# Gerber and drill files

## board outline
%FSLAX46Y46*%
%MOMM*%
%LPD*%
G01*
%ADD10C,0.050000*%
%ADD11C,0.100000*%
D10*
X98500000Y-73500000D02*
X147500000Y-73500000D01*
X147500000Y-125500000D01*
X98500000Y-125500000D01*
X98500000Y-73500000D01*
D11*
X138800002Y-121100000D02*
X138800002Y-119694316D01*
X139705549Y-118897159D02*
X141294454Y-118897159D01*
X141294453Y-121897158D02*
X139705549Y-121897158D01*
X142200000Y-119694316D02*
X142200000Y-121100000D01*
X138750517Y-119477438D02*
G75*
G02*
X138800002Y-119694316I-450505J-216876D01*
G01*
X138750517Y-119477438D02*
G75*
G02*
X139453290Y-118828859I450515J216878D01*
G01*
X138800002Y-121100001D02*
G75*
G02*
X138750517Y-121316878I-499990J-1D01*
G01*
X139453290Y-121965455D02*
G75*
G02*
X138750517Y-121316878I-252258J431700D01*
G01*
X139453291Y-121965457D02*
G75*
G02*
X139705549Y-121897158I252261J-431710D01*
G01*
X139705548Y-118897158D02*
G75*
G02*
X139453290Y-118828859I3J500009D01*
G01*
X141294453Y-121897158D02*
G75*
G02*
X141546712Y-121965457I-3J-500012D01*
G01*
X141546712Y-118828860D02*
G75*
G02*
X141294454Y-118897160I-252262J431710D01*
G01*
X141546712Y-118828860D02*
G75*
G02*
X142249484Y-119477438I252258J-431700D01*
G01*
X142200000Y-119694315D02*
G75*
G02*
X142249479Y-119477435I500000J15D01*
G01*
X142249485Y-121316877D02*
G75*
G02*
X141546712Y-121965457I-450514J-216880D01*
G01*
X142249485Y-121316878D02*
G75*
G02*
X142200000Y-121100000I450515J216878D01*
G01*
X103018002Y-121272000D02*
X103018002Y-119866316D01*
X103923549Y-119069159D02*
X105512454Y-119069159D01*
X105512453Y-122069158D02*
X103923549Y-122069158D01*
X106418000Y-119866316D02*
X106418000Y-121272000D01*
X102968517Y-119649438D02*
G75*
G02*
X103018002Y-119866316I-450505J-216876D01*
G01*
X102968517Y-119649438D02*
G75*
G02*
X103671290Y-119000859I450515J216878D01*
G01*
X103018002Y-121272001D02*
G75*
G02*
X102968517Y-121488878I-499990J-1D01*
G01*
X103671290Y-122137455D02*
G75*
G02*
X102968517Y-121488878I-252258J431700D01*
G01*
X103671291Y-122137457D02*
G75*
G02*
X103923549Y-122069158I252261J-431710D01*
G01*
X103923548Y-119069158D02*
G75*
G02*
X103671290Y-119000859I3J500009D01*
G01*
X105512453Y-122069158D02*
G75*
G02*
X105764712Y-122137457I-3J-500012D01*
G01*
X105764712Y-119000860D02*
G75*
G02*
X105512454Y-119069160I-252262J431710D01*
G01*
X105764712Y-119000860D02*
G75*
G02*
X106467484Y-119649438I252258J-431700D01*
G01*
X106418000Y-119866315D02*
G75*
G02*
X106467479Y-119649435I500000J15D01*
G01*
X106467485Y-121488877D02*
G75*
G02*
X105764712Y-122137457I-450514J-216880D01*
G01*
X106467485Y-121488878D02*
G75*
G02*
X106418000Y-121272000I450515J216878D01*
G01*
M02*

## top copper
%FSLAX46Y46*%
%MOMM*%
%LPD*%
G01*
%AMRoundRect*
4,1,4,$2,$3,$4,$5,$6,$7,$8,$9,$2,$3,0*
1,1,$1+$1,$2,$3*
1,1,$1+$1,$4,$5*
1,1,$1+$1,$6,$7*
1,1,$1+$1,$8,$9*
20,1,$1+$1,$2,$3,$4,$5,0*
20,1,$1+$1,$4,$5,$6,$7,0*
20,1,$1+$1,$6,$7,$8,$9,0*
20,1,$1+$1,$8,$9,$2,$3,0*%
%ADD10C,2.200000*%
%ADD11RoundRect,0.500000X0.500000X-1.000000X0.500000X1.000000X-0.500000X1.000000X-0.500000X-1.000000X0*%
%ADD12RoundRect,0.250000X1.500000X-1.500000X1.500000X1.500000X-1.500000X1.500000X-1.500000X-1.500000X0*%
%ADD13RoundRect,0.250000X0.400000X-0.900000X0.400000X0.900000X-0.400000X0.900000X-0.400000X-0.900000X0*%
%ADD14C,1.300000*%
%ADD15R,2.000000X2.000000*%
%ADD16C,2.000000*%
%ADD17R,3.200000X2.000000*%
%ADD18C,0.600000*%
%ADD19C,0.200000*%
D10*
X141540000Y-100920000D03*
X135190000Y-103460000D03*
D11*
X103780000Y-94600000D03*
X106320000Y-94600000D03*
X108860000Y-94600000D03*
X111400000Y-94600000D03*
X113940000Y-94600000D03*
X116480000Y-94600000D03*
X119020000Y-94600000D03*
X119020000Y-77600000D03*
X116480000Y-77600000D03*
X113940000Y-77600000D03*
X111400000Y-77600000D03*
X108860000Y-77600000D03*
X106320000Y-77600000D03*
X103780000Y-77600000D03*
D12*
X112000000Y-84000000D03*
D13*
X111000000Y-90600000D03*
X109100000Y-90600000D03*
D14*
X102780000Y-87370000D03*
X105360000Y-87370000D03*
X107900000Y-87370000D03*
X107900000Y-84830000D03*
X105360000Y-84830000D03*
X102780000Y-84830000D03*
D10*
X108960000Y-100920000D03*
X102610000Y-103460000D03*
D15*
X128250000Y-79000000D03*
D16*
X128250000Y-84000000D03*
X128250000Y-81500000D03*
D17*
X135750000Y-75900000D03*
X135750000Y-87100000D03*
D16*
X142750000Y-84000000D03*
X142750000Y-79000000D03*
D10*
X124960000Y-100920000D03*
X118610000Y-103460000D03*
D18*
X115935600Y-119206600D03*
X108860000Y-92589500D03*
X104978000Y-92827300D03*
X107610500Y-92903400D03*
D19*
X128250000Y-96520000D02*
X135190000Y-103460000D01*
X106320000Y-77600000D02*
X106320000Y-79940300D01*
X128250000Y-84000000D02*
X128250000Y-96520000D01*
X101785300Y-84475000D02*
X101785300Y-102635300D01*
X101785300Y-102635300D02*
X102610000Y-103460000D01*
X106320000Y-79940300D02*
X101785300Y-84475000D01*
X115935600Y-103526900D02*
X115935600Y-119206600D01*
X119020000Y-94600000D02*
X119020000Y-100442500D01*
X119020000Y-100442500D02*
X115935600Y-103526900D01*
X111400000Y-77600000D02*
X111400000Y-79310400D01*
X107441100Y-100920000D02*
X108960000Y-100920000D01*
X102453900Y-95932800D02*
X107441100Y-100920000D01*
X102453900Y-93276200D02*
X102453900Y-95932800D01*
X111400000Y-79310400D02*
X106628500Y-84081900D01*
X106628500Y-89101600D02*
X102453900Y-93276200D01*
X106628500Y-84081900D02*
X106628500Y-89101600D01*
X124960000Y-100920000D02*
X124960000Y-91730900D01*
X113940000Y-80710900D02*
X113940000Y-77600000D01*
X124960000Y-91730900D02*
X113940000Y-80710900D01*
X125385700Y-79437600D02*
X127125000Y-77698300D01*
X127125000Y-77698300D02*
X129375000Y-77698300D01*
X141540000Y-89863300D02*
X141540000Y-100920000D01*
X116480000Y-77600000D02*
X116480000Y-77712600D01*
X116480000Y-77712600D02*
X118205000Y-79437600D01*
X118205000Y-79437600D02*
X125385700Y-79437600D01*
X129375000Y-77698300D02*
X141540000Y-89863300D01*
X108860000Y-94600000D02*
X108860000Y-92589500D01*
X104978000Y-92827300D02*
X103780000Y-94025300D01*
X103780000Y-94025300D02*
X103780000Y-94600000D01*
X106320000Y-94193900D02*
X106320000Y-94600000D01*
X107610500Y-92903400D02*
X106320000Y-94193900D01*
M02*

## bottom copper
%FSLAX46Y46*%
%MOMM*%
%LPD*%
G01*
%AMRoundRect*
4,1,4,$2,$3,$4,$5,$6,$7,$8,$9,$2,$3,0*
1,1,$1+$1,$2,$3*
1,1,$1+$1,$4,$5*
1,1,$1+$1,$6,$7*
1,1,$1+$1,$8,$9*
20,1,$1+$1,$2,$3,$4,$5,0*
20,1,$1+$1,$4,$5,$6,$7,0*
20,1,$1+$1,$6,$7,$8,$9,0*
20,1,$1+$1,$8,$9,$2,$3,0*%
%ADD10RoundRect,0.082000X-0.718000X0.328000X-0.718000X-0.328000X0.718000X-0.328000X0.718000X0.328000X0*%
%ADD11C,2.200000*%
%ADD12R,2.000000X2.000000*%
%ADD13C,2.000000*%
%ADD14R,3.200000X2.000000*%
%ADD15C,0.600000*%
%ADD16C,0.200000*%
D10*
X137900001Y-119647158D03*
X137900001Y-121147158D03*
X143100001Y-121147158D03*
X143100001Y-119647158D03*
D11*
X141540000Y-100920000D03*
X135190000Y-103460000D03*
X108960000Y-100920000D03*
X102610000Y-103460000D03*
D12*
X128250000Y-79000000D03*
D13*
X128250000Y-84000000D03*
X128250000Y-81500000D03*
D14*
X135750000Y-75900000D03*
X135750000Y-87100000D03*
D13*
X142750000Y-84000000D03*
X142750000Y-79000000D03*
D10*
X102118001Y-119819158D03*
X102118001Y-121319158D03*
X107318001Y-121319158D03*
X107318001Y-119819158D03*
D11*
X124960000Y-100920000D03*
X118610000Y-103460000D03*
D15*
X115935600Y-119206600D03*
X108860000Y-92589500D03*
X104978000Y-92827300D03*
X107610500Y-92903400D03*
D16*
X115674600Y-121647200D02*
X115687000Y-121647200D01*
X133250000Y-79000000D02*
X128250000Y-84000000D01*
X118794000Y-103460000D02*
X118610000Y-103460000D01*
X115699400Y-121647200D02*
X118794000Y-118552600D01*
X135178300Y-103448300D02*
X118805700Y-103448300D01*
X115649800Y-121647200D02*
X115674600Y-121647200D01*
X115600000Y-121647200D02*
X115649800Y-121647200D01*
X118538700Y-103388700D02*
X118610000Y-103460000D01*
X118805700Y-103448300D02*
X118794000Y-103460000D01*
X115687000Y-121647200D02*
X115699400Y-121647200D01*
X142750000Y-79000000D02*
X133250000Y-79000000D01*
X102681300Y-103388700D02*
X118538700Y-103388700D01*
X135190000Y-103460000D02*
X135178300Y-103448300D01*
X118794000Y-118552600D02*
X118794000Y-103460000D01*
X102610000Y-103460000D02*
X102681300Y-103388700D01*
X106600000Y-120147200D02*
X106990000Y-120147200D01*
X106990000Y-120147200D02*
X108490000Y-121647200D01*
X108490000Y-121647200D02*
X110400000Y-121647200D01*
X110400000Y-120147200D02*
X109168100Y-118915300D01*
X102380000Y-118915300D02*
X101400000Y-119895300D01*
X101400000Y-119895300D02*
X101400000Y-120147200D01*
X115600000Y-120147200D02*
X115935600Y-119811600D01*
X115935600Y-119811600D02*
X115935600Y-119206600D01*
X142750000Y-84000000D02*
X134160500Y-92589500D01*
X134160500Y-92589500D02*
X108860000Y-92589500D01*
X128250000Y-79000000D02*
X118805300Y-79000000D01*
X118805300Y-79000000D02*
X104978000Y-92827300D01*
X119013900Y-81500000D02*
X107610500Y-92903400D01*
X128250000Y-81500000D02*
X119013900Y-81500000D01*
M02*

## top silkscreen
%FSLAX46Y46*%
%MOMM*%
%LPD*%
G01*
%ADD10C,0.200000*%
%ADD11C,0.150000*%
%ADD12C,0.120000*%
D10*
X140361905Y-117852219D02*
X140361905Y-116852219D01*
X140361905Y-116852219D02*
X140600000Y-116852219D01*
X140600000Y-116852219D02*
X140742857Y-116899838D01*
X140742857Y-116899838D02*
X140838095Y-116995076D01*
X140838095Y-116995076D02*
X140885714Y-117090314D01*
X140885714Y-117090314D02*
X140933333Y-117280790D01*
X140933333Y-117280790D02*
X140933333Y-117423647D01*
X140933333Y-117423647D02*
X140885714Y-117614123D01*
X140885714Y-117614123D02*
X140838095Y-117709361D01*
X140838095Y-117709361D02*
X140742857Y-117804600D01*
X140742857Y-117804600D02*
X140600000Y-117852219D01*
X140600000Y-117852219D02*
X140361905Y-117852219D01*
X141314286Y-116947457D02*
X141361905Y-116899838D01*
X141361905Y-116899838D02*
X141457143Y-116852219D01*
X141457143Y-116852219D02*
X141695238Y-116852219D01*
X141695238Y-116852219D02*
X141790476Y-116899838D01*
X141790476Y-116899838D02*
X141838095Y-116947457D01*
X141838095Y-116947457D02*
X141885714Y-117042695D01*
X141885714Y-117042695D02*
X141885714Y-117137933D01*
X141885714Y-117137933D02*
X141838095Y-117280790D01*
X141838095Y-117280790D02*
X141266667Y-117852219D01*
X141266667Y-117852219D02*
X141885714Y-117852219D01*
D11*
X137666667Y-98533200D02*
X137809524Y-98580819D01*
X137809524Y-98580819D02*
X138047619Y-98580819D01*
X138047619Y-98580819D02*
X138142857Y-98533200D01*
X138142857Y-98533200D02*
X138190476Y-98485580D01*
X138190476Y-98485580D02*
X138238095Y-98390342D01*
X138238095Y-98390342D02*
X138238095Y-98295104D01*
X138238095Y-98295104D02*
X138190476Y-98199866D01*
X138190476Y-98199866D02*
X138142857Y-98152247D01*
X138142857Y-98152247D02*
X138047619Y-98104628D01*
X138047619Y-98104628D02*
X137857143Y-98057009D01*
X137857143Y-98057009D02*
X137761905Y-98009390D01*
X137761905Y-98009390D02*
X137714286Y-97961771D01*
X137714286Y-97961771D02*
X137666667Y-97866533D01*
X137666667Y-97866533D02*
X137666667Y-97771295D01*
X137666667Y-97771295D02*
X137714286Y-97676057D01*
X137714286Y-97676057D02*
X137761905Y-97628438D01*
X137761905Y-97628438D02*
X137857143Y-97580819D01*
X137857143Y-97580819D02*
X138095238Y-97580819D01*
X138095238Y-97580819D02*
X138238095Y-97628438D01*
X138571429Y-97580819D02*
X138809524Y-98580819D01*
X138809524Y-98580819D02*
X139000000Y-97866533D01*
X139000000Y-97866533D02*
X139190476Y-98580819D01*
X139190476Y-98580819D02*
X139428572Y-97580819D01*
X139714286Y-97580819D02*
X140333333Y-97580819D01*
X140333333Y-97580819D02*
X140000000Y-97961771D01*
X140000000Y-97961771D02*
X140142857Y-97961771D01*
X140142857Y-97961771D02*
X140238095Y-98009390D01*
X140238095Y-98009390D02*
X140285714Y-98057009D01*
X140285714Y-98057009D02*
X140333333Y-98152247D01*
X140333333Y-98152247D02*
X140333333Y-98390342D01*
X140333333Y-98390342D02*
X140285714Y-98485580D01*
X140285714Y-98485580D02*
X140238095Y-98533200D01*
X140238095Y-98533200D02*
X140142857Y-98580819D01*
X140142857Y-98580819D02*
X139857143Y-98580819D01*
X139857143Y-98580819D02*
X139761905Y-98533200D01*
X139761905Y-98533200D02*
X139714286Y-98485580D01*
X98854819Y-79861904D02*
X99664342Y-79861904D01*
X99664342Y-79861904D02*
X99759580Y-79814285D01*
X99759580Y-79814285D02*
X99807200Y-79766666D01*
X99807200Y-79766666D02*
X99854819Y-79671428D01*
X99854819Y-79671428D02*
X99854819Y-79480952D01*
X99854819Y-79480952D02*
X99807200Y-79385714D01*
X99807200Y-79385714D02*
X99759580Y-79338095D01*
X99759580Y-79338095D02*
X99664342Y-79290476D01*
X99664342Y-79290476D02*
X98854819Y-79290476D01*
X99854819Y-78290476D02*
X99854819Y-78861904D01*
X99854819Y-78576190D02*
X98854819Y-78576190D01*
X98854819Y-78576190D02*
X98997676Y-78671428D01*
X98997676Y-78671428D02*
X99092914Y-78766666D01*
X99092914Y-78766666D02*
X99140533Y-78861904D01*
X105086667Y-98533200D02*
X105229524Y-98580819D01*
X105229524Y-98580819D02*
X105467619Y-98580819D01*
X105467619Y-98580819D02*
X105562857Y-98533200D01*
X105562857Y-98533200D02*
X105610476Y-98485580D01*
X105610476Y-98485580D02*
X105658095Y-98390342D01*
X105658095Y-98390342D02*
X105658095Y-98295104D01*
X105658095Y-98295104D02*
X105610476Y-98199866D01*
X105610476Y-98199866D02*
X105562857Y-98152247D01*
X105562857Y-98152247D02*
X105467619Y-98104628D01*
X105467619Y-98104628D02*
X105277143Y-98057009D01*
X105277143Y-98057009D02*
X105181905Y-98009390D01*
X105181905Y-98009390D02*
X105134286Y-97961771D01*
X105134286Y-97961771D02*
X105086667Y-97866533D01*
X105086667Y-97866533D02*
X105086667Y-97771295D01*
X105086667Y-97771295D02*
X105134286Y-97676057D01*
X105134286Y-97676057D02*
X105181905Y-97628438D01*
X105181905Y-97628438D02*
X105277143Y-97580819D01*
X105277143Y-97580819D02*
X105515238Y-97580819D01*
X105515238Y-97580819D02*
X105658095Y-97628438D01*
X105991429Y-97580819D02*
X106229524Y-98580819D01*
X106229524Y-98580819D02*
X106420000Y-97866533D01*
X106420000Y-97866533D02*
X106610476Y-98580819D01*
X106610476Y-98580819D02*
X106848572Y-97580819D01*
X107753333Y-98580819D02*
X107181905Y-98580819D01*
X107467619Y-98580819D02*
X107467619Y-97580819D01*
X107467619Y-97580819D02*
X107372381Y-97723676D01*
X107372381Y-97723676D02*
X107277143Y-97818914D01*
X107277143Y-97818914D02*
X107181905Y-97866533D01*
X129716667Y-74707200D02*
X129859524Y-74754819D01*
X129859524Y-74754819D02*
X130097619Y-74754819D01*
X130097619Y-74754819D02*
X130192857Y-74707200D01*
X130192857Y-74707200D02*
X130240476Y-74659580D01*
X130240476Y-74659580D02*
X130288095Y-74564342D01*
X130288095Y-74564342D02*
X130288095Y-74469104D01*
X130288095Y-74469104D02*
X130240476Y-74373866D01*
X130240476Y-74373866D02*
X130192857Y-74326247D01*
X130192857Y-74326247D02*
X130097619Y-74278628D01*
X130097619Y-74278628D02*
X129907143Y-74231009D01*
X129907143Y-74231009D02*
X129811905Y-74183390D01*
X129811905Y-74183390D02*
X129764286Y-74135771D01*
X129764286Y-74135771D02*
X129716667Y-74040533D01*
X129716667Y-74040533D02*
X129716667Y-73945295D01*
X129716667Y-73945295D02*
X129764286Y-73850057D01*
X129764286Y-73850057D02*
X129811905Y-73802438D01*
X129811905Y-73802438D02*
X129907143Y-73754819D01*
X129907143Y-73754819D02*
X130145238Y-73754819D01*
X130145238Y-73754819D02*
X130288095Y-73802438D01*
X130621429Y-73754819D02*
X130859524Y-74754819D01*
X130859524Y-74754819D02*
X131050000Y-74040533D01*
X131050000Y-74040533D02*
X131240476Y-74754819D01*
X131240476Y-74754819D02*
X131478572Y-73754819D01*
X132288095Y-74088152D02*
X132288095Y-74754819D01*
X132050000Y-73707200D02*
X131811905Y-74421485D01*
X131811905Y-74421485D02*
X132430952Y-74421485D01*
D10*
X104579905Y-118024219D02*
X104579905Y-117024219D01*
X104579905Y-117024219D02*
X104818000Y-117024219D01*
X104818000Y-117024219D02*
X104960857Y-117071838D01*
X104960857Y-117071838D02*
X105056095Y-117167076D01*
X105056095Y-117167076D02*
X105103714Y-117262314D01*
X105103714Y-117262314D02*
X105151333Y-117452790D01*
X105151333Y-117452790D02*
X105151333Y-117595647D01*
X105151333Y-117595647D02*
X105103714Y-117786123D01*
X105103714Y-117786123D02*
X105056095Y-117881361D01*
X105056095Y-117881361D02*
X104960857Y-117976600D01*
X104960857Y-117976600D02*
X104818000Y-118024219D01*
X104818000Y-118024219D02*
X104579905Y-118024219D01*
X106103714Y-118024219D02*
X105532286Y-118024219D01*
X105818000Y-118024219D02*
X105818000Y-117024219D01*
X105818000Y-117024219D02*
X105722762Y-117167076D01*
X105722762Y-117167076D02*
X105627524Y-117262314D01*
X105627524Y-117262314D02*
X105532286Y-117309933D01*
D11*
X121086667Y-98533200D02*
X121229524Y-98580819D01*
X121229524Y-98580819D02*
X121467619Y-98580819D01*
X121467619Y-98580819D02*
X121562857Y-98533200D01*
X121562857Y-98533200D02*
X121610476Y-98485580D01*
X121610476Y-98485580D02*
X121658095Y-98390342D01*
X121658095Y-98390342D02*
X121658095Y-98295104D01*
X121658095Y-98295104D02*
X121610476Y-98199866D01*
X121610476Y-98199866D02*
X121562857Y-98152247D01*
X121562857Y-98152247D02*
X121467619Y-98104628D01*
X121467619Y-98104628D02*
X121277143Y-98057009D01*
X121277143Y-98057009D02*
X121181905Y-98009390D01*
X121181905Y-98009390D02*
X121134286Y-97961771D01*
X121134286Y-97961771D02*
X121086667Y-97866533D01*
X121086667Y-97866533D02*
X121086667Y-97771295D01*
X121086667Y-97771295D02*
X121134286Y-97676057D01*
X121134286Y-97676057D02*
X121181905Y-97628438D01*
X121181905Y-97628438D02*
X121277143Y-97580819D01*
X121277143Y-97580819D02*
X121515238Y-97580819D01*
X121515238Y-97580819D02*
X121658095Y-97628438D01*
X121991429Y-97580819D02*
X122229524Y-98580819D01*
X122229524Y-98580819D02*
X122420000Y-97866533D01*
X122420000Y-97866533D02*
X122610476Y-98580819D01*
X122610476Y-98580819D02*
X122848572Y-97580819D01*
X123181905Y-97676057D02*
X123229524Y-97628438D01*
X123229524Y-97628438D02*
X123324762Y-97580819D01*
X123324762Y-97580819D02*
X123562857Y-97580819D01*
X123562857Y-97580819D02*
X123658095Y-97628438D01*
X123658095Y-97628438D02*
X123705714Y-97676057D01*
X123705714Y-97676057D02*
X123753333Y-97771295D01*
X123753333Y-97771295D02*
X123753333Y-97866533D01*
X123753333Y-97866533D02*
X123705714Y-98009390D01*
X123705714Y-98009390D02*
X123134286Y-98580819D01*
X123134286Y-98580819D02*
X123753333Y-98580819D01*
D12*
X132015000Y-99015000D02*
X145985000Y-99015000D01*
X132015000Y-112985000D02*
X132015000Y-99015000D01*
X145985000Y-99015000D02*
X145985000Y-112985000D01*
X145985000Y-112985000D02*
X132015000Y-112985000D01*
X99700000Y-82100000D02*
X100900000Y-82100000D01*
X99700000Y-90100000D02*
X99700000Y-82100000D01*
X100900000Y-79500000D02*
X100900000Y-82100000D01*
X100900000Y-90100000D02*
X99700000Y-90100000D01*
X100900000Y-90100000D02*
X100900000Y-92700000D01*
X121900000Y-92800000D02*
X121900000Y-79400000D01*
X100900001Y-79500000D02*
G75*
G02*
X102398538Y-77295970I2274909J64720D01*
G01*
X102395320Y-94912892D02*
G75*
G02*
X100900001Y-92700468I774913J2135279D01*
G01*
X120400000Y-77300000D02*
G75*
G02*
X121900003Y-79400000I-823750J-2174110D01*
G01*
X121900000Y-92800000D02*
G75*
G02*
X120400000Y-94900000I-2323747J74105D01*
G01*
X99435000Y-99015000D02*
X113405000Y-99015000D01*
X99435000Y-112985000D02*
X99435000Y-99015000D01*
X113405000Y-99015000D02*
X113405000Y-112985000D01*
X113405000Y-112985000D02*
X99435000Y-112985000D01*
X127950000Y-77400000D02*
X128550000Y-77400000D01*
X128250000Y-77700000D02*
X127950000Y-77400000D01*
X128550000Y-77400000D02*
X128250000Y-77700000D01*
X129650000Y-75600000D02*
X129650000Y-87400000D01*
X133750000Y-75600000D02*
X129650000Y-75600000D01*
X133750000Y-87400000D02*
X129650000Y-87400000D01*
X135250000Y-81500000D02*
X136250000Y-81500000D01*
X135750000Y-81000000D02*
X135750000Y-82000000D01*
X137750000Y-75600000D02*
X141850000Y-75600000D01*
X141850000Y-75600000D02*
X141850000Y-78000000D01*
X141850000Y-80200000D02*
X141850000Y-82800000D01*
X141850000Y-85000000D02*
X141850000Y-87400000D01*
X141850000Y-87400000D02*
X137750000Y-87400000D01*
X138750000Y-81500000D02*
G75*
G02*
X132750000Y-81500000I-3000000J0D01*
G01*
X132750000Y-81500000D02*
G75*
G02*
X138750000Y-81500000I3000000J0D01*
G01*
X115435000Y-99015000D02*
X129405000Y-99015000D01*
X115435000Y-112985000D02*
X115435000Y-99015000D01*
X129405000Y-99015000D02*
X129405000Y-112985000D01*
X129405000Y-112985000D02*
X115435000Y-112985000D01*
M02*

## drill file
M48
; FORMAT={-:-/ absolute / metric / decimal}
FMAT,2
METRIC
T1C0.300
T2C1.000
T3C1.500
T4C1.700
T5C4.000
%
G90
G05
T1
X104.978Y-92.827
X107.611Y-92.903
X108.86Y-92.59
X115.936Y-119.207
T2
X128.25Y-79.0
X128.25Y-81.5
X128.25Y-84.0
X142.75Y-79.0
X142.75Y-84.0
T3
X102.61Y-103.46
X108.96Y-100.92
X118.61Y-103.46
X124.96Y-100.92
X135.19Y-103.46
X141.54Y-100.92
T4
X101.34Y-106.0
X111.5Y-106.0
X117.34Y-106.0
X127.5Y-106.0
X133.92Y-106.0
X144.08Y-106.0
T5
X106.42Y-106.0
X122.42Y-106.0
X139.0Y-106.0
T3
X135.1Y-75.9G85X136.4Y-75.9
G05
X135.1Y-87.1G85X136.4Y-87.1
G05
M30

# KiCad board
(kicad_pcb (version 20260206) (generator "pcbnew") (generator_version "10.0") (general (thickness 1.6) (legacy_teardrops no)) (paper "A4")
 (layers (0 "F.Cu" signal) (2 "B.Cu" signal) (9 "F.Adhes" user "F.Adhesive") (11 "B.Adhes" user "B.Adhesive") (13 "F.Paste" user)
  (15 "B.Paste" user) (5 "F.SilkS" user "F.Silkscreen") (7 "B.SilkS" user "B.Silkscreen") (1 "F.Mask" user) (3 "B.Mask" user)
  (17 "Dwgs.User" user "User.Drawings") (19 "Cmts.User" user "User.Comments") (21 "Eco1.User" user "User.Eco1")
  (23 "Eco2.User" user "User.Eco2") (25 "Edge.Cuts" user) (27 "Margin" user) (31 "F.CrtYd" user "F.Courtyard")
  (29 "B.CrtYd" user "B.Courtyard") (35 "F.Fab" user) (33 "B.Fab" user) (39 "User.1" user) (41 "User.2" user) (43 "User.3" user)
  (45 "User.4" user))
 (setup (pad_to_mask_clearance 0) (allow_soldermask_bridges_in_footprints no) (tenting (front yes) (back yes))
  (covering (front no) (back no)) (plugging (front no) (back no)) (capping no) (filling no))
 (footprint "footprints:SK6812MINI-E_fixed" (layer "F.Cu") (at 140.5 120.5)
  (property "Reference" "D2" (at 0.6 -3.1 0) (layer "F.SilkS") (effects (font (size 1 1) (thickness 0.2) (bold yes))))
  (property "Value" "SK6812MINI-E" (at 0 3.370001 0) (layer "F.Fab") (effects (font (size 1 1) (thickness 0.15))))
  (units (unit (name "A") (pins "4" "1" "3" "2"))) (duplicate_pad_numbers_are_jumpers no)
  (fp_line (start -1.699998 0.6) (end -1.699998 -0.805684) (stroke (width 0.1) (type solid)) (layer "Edge.Cuts"))
  (fp_line (start -0.794451 -1.602841) (end 0.794454 -1.602841) (stroke (width 0.1) (type solid)) (layer "Edge.Cuts"))
  (fp_line (start 0.794453 1.397158) (end -0.794451 1.397158) (stroke (width 0.1) (type solid)) (layer "Edge.Cuts"))
  (fp_line (start 1.7 -0.805684) (end 1.7 0.6) (stroke (width 0.1) (type solid)) (layer "Edge.Cuts"))
  (fp_arc (start -1.749483 -1.022562) (mid -1.712526 -0.91691) (end -1.699998 -0.805684) (stroke (width 0.1) (type solid))
   (layer "Edge.Cuts"))
  (fp_arc (start -1.749483 -1.022562) (mid -1.63807 -1.606877) (end -1.04671 -1.671141) (stroke (width 0.1) (type solid))
   (layer "Edge.Cuts"))
  (fp_arc (start -1.699998 0.600001) (mid -1.712526 0.711226) (end -1.749483 0.816878) (stroke (width 0.1) (type solid)) (layer "Edge.Cuts"))
  (fp_arc (start -1.04671 1.465455) (mid -1.638069 1.401192) (end -1.749483 0.816878) (stroke (width 0.1) (type solid)) (layer "Edge.Cuts"))
  (fp_arc (start -1.046709 1.465457) (mid -0.925121 1.414535) (end -0.794451 1.397158) (stroke (width 0.1) (type solid)) (layer "Edge.Cuts"))
  (fp_arc (start -0.794452 -1.602842) (mid -0.925122 -1.620219) (end -1.04671 -1.671141) (stroke (width 0.1) (type solid))
   (layer "Edge.Cuts"))
  (fp_arc (start 0.794453 1.397158) (mid 0.925124 1.414535) (end 1.046712 1.465457) (stroke (width 0.1) (type solid)) (layer "Edge.Cuts"))
  (fp_arc (start 1.046712 -1.67114) (mid 0.925124 -1.620218) (end 0.794454 -1.602841) (stroke (width 0.1) (type solid)) (layer "Edge.Cuts"))
  (fp_arc (start 1.046712 -1.67114) (mid 1.638072 -1.606876) (end 1.749485 -1.022562) (stroke (width 0.1) (type solid)) (layer "Edge.Cuts"))
  (fp_arc (start 1.7 -0.805685) (mid 1.712528 -0.91691) (end 1.749485 -1.022562) (stroke (width 0.1) (type solid)) (layer "Edge.Cuts"))
  (fp_arc (start 1.749485 0.816877) (mid 1.638073 1.401193) (end 1.046712 1.465457) (stroke (width 0.1) (type solid)) (layer "Edge.Cuts"))
  (fp_arc (start 1.749485 0.816878) (mid 1.712528 0.711226) (end 1.7 0.6) (stroke (width 0.1) (type solid)) (layer "Edge.Cuts"))
  (pad "1" smd roundrect (at -2.599999 -0.852842 270) (size 0.82 1.6) (layers "B.Cu" "B.Mask" "B.Paste") (roundrect_rratio 0.1) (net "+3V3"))
  (pad "2" smd roundrect (at -2.599999 0.647158 270) (size 0.82 1.6) (layers "B.Cu" "B.Mask" "B.Paste") (roundrect_rratio 0.1)
   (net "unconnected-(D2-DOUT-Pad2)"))
  (pad "3" smd roundrect (at 2.600001 0.647158 270) (size 0.82 1.6) (layers "B.Cu" "B.Mask" "B.Paste") (roundrect_rratio 0.1) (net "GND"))
  (pad "4" smd roundrect (at 2.600001 -0.852842 270) (size 0.82 1.6) (layers "B.Cu" "B.Mask" "B.Paste") (roundrect_rratio 0.1)
   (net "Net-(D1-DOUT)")))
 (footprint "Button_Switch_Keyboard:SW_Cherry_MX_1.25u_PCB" (layer "F.Cu") (at 141.54 100.92)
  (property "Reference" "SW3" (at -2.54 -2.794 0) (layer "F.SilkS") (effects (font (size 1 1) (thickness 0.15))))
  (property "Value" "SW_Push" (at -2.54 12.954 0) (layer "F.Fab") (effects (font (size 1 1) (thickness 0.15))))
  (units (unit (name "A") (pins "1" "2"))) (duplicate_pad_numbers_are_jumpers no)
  (fp_line (start -9.525 -1.905) (end 4.445 -1.905) (stroke (width 0.12) (type solid)) (layer "F.SilkS"))
  (fp_line (start -9.525 12.065) (end -9.525 -1.905) (stroke (width 0.12) (type solid)) (layer "F.SilkS"))
  (fp_line (start 4.445 -1.905) (end 4.445 12.065) (stroke (width 0.12) (type solid)) (layer "F.SilkS"))
  (fp_line (start 4.445 12.065) (end -9.525 12.065) (stroke (width 0.12) (type solid)) (layer "F.SilkS"))
  (pad "" np_thru_hole circle (at -7.62 5.08) (size 1.7 1.7) (drill 1.7) (layers "*.Cu" "*.Mask"))
  (pad "" np_thru_hole circle (at -2.54 5.08) (size 4 4) (drill 4) (layers "*.Cu" "*.Mask"))
  (pad "" np_thru_hole circle (at 2.54 5.08) (size 1.7 1.7) (drill 1.7) (layers "*.Cu" "*.Mask"))
  (pad "1" thru_hole circle (at 0 0) (size 2.2 2.2) (drill 1.5) (layers "*.Cu" "*.Mask") (remove_unused_layers no)
   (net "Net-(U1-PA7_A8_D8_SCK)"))
  (pad "2" thru_hole circle (at -6.35 2.54) (size 2.2 2.2) (drill 1.5) (layers "*.Cu" "*.Mask") (remove_unused_layers no) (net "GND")))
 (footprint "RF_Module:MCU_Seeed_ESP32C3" (layer "F.Cu") (at 111.4 86.1 90)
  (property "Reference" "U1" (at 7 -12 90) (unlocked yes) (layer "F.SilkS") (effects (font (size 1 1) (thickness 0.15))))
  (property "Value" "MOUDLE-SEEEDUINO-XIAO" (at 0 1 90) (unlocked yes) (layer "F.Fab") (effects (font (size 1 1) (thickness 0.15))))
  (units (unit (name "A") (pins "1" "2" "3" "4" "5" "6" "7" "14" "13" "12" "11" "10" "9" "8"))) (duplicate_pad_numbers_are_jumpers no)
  (fp_line (start 4 -11.7) (end 4 -10.5) (stroke (width 0.12) (type default)) (layer "F.SilkS"))
  (fp_line (start -4 -11.7) (end 4 -11.7) (stroke (width 0.12) (type default)) (layer "F.SilkS"))
  (fp_line (start 6.6 -10.5) (end 4 -10.5) (stroke (width 0.12) (type default)) (layer "F.SilkS"))
  (fp_line (start -4 -10.5) (end -4 -11.7) (stroke (width 0.12) (type default)) (layer "F.SilkS"))
  (fp_line (start -4 -10.5) (end -6.6 -10.5) (stroke (width 0.12) (type default)) (layer "F.SilkS"))
  (fp_line (start -6.7 10.5) (end 6.7 10.5) (stroke (width 0.12) (type default)) (layer "F.SilkS"))
  (fp_arc (start 6.6 -10.499999) (mid 7.944325 -10.107116) (end 8.804034 -9.001464) (stroke (width 0.12) (type default)) (layer "F.SilkS"))
  (fp_arc (start -8.812892 -9.00468) (mid -7.949609 -10.111769) (end -6.600468 -10.499999) (stroke (width 0.12) (type default))
   (layer "F.SilkS"))
  (fp_arc (start 8.8 9) (mid 7.977232 10.068125) (end 6.7 10.5) (stroke (width 0.12) (type default)) (layer "F.SilkS"))
  (fp_arc (start -6.7 10.5) (mid -7.977232 10.068125) (end -8.8 9) (stroke (width 0.12) (type default)) (layer "F.SilkS"))
  (pad "" smd roundrect (at 1.1 -0.4 90) (size 1.5 1.5) (layers "F.Paste") (roundrect_rratio 0.1666666667))
  (pad "" smd roundrect (at 1.1 1.6 90) (size 1.5 1.5) (layers "F.Paste") (roundrect_rratio 0.1666666667))
  (pad "" smd roundrect (at 3.1 -0.4 90) (size 1.5 1.5) (layers "F.Paste") (roundrect_rratio 0.1666666667))
  (pad "" smd roundrect (at 3.1 1.6 90) (size 1.5 1.5) (layers "F.Paste") (roundrect_rratio 0.1666666667))
  (pad "1" smd roundrect (at -8.5 -7.62 90) (size 3 2) (layers "F.Cu" "F.Mask" "F.Paste") (roundrect_rratio 0.25)
   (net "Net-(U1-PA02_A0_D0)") (thermal_bridge_angle 45))
  (pad "2" smd roundrect (at -8.5 -5.08 90) (size 3 2) (layers "F.Cu" "F.Mask" "F.Paste") (roundrect_rratio 0.25) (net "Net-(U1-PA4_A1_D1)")
   (thermal_bridge_angle 45))
  (pad "3" smd roundrect (at -8.5 -2.54 90) (size 3 2) (layers "F.Cu" "F.Mask" "F.Paste") (roundrect_rratio 0.25)
   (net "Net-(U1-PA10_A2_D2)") (thermal_bridge_angle 45))
  (pad "4" smd roundrect (at -8.5 0 90) (size 3 2) (layers "F.Cu" "F.Mask" "F.Paste") (roundrect_rratio 0.25)
   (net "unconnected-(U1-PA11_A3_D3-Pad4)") (thermal_bridge_angle 45))
  (pad "5" smd roundrect (at -8.5 2.54 90) (size 3 2) (layers "F.Cu" "F.Mask" "F.Paste") (roundrect_rratio 0.25)
   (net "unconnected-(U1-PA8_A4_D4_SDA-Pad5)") (thermal_bridge_angle 45))
  (pad "6" smd roundrect (at -8.5 5.08 90) (size 3 2) (layers "F.Cu" "F.Mask" "F.Paste") (roundrect_rratio 0.25)
   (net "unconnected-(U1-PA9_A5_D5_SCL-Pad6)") (thermal_bridge_angle 45))
  (pad "7" smd roundrect (at -8.5 7.62 90) (size 3 2) (layers "F.Cu" "F.Mask" "F.Paste") (roundrect_rratio 0.25) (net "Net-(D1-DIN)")
   (thermal_bridge_angle 45))
  (pad "8" smd roundrect (at 8.5 7.62 90) (size 3 2) (layers "F.Cu" "F.Mask" "F.Paste") (roundrect_rratio 0.25)
   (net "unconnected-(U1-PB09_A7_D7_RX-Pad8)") (thermal_bridge_angle 45))
  (pad "9" smd roundrect (at 8.5 5.08 90) (size 3 2) (layers "F.Cu" "F.Mask" "F.Paste") (roundrect_rratio 0.25)
   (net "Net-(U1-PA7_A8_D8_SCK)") (thermal_bridge_angle 45))
  (pad "10" smd roundrect (at 8.5 2.54 90) (size 3 2) (layers "F.Cu" "F.Mask" "F.Paste") (roundrect_rratio 0.25)
   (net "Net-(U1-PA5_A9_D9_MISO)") (thermal_bridge_angle 45))
  (pad "11" smd roundrect (at 8.5 0 90) (size 3 2) (layers "F.Cu" "F.Mask" "F.Paste") (roundrect_rratio 0.25)
   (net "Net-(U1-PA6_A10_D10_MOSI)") (thermal_bridge_angle 45))
  (pad "12" smd roundrect (at 8.5 -2.54 90) (size 3 2) (layers "F.Cu" "F.Mask" "F.Paste") (roundrect_rratio 0.25)
   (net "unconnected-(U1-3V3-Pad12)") (thermal_bridge_angle 45))
  (pad "13" smd roundrect (at 8.5 -5.08 90) (size 3 2) (layers "F.Cu" "F.Mask" "F.Paste") (roundrect_rratio 0.25) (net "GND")
   (thermal_bridge_angle 45))
  (pad "14" smd roundrect (at 8.5 -7.62 90) (size 3 2) (layers "F.Cu" "F.Mask" "F.Paste") (roundrect_rratio 0.25)
   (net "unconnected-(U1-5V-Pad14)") (thermal_bridge_angle 45))
  (pad "15" smd roundrect (at 2.1 0.6 90) (size 3.5 3.5) (layers "F.Cu" "F.Mask") (roundrect_rratio 0.07142857143))
  (pad "16" smd roundrect (at -4.5 -0.4 90) (size 2.3 1.3) (layers "F.Cu" "F.Mask" "F.Paste") (roundrect_rratio 0.1923076923))
  (pad "17" smd roundrect (at -4.5 -2.3 90) (size 2.3 1.3) (layers "F.Cu" "F.Mask" "F.Paste") (roundrect_rratio 0.1923076923))
  (pad "18" smd circle (at -1.27 -8.62 90) (size 1.3 1.3) (layers "F.Cu" "F.Mask" "F.Paste"))
  (pad "19" smd circle (at -1.27 -6.04 90) (size 1.3 1.3) (layers "F.Cu" "F.Mask" "F.Paste"))
  (pad "20" smd circle (at -1.27 -3.5 90) (size 1.3 1.3) (layers "F.Cu" "F.Mask" "F.Paste"))
  (pad "21" smd circle (at 1.27 -3.5 90) (size 1.3 1.3) (layers "F.Cu" "F.Mask" "F.Paste"))
  (pad "22" smd circle (at 1.27 -6.04 90) (size 1.3 1.3) (layers "F.Cu" "F.Mask" "F.Paste"))
  (pad "23" smd circle (at 1.27 -8.62 90) (size 1.3 1.3) (layers "F.Cu" "F.Mask" "F.Paste")))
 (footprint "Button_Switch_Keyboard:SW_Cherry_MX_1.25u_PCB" (layer "F.Cu") (at 108.96 100.92)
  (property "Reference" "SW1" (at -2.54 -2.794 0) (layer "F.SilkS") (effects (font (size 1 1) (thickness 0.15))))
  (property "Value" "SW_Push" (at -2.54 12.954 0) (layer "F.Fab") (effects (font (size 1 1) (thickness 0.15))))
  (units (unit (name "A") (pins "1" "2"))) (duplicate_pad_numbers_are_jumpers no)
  (fp_line (start -9.525 -1.905) (end 4.445 -1.905) (stroke (width 0.12) (type solid)) (layer "F.SilkS"))
  (fp_line (start -9.525 12.065) (end -9.525 -1.905) (stroke (width 0.12) (type solid)) (layer "F.SilkS"))
  (fp_line (start 4.445 -1.905) (end 4.445 12.065) (stroke (width 0.12) (type solid)) (layer "F.SilkS"))
  (fp_line (start 4.445 12.065) (end -9.525 12.065) (stroke (width 0.12) (type solid)) (layer "F.SilkS"))
  (pad "" np_thru_hole circle (at -7.62 5.08) (size 1.7 1.7) (drill 1.7) (layers "*.Cu" "*.Mask"))
  (pad "" np_thru_hole circle (at -2.54 5.08) (size 4 4) (drill 4) (layers "*.Cu" "*.Mask"))
  (pad "" np_thru_hole circle (at 2.54 5.08) (size 1.7 1.7) (drill 1.7) (layers "*.Cu" "*.Mask"))
  (pad "1" thru_hole circle (at 0 0) (size 2.2 2.2) (drill 1.5) (layers "*.Cu" "*.Mask") (remove_unused_layers no)
   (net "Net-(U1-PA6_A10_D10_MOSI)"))
  (pad "2" thru_hole circle (at -6.35 2.54) (size 2.2 2.2) (drill 1.5) (layers "*.Cu" "*.Mask") (remove_unused_layers no) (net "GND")))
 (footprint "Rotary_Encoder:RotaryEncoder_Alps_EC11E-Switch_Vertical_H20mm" (layer "F.Cu") (at 128.25 79)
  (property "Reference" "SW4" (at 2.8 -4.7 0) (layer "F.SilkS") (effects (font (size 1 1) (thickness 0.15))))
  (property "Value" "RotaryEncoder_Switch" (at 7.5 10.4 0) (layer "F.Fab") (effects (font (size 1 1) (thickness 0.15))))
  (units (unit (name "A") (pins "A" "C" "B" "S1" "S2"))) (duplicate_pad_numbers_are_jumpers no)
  (fp_line (start -0.3 -1.6) (end 0.3 -1.6) (stroke (width 0.12) (type solid)) (layer "F.SilkS"))
  (fp_line (start 0 -1.3) (end -0.3 -1.6) (stroke (width 0.12) (type solid)) (layer "F.SilkS"))
  (fp_line (start 0.3 -1.6) (end 0 -1.3) (stroke (width 0.12) (type solid)) (layer "F.SilkS"))
  (fp_line (start 1.4 -3.4) (end 1.4 8.4) (stroke (width 0.12) (type solid)) (layer "F.SilkS"))
  (fp_line (start 5.5 -3.4) (end 1.4 -3.4) (stroke (width 0.12) (type solid)) (layer "F.SilkS"))
  (fp_line (start 5.5 8.4) (end 1.4 8.4) (stroke (width 0.12) (type solid)) (layer "F.SilkS"))
  (fp_line (start 7 2.5) (end 8 2.5) (stroke (width 0.12) (type solid)) (layer "F.SilkS"))
  (fp_line (start 7.5 2) (end 7.5 3) (stroke (width 0.12) (type solid)) (layer "F.SilkS"))
  (fp_line (start 9.5 -3.4) (end 13.6 -3.4) (stroke (width 0.12) (type solid)) (layer "F.SilkS"))
  (fp_line (start 13.6 -3.4) (end 13.6 -1) (stroke (width 0.12) (type solid)) (layer "F.SilkS"))
  (fp_line (start 13.6 1.2) (end 13.6 3.8) (stroke (width 0.12) (type solid)) (layer "F.SilkS"))
  (fp_line (start 13.6 6) (end 13.6 8.4) (stroke (width 0.12) (type solid)) (layer "F.SilkS"))
  (fp_line (start 13.6 8.4) (end 9.5 8.4) (stroke (width 0.12) (type solid)) (layer "F.SilkS"))
  (fp_circle (center 7.5 2.5) (end 10.5 2.5) (stroke (width 0.12) (type solid)) (fill no) (layer "F.SilkS"))
  (pad "A" thru_hole rect (at 0 0) (size 2 2) (drill 1) (layers "*.Cu" "*.Mask") (remove_unused_layers no) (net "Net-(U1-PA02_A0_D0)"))
  (pad "B" thru_hole circle (at 0 5) (size 2 2) (drill 1) (layers "*.Cu" "*.Mask") (remove_unused_layers no) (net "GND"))
  (pad "C" thru_hole circle (at 0 2.5) (size 2 2) (drill 1) (layers "*.Cu" "*.Mask") (remove_unused_layers no) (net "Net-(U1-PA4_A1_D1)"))
  (pad "MP" thru_hole rect (at 7.5 -3.1) (size 3.2 2) (drill oval 2.8 1.5) (layers "*.Cu" "*.Mask") (remove_unused_layers no))
  (pad "MP" thru_hole rect (at 7.5 8.1) (size 3.2 2) (drill oval 2.8 1.5) (layers "*.Cu" "*.Mask") (remove_unused_layers no))
  (pad "S1" thru_hole circle (at 14.5 5) (size 2 2) (drill 1) (layers "*.Cu" "*.Mask") (remove_unused_layers no) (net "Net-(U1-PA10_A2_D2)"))
  (pad "S2" thru_hole circle (at 14.5 0) (size 2 2) (drill 1) (layers "*.Cu" "*.Mask") (remove_unused_layers no) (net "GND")))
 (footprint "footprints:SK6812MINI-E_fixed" (layer "F.Cu") (at 104.718 120.672)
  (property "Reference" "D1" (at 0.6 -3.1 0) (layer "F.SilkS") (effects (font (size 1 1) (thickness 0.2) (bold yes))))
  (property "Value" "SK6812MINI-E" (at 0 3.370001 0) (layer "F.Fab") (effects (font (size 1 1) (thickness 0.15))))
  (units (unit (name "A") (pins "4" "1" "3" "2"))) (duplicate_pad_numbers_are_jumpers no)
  (fp_line (start -1.699998 0.6) (end -1.699998 -0.805684) (stroke (width 0.1) (type solid)) (layer "Edge.Cuts"))
  (fp_line (start -0.794451 -1.602841) (end 0.794454 -1.602841) (stroke (width 0.1) (type solid)) (layer "Edge.Cuts"))
  (fp_line (start 0.794453 1.397158) (end -0.794451 1.397158) (stroke (width 0.1) (type solid)) (layer "Edge.Cuts"))
  (fp_line (start 1.7 -0.805684) (end 1.7 0.6) (stroke (width 0.1) (type solid)) (layer "Edge.Cuts"))
  (fp_arc (start -1.749483 -1.022562) (mid -1.712526 -0.91691) (end -1.699998 -0.805684) (stroke (width 0.1) (type solid))
   (layer "Edge.Cuts"))
  (fp_arc (start -1.749483 -1.022562) (mid -1.63807 -1.606877) (end -1.04671 -1.671141) (stroke (width 0.1) (type solid))
   (layer "Edge.Cuts"))
  (fp_arc (start -1.699998 0.600001) (mid -1.712526 0.711226) (end -1.749483 0.816878) (stroke (width 0.1) (type solid)) (layer "Edge.Cuts"))
  (fp_arc (start -1.04671 1.465455) (mid -1.638069 1.401192) (end -1.749483 0.816878) (stroke (width 0.1) (type solid)) (layer "Edge.Cuts"))
  (fp_arc (start -1.046709 1.465457) (mid -0.925121 1.414535) (end -0.794451 1.397158) (stroke (width 0.1) (type solid)) (layer "Edge.Cuts"))
  (fp_arc (start -0.794452 -1.602842) (mid -0.925122 -1.620219) (end -1.04671 -1.671141) (stroke (width 0.1) (type solid))
   (layer "Edge.Cuts"))
  (fp_arc (start 0.794453 1.397158) (mid 0.925124 1.414535) (end 1.046712 1.465457) (stroke (width 0.1) (type solid)) (layer "Edge.Cuts"))
  (fp_arc (start 1.046712 -1.67114) (mid 0.925124 -1.620218) (end 0.794454 -1.602841) (stroke (width 0.1) (type solid)) (layer "Edge.Cuts"))
  (fp_arc (start 1.046712 -1.67114) (mid 1.638072 -1.606876) (end 1.749485 -1.022562) (stroke (width 0.1) (type solid)) (layer "Edge.Cuts"))
  (fp_arc (start 1.7 -0.805685) (mid 1.712528 -0.91691) (end 1.749485 -1.022562) (stroke (width 0.1) (type solid)) (layer "Edge.Cuts"))
  (fp_arc (start 1.749485 0.816877) (mid 1.638073 1.401193) (end 1.046712 1.465457) (stroke (width 0.1) (type solid)) (layer "Edge.Cuts"))
  (fp_arc (start 1.749485 0.816878) (mid 1.712528 0.711226) (end 1.7 0.6) (stroke (width 0.1) (type solid)) (layer "Edge.Cuts"))
  (pad "1" smd roundrect (at -2.599999 -0.852842 270) (size 0.82 1.6) (layers "B.Cu" "B.Mask" "B.Paste") (roundrect_rratio 0.1) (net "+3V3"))
  (pad "2" smd roundrect (at -2.599999 0.647158 270) (size 0.82 1.6) (layers "B.Cu" "B.Mask" "B.Paste") (roundrect_rratio 0.1)
   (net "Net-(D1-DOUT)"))
  (pad "3" smd roundrect (at 2.600001 0.647158 270) (size 0.82 1.6) (layers "B.Cu" "B.Mask" "B.Paste") (roundrect_rratio 0.1) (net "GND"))
  (pad "4" smd roundrect (at 2.600001 -0.852842 270) (size 0.82 1.6) (layers "B.Cu" "B.Mask" "B.Paste") (roundrect_rratio 0.1)
   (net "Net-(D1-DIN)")))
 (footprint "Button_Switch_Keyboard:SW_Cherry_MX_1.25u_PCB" (layer "F.Cu") (at 124.96 100.92)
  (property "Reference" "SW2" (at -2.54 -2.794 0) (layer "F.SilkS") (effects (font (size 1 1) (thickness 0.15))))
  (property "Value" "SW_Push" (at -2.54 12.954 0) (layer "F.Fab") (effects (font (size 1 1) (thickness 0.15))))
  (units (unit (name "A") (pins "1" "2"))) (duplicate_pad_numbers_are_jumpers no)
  (fp_line (start -9.525 -1.905) (end 4.445 -1.905) (stroke (width 0.12) (type solid)) (layer "F.SilkS"))
  (fp_line (start -9.525 12.065) (end -9.525 -1.905) (stroke (width 0.12) (type solid)) (layer "F.SilkS"))
  (fp_line (start 4.445 -1.905) (end 4.445 12.065) (stroke (width 0.12) (type solid)) (layer "F.SilkS"))
  (fp_line (start 4.445 12.065) (end -9.525 12.065) (stroke (width 0.12) (type solid)) (layer "F.SilkS"))
  (pad "" np_thru_hole circle (at -7.62 5.08) (size 1.7 1.7) (drill 1.7) (layers "*.Cu" "*.Mask"))
  (pad "" np_thru_hole circle (at -2.54 5.08) (size 4 4) (drill 4) (layers "*.Cu" "*.Mask"))
  (pad "" np_thru_hole circle (at 2.54 5.08) (size 1.7 1.7) (drill 1.7) (layers "*.Cu" "*.Mask"))
  (pad "1" thru_hole circle (at 0 0) (size 2.2 2.2) (drill 1.5) (layers "*.Cu" "*.Mask") (remove_unused_layers no)
   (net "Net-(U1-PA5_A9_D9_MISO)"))
  (pad "2" thru_hole circle (at -6.35 2.54) (size 2.2 2.2) (drill 1.5) (layers "*.Cu" "*.Mask") (remove_unused_layers no) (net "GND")))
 (gr_rect (start 98.5 73.5) (end 147.5 125.5) (stroke (width 0.05) (type default)) (fill no) (layer "Edge.Cuts"))
 (segment (start 128.25 96.52) (end 135.19 103.46) (width 0.2) (layer "F.Cu") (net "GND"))
 (segment (start 106.32 77.6) (end 106.32 79.9403) (width 0.2) (layer "F.Cu") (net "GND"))
 (segment (start 128.25 84) (end 128.25 96.52) (width 0.2) (layer "F.Cu") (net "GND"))
 (segment (start 101.7853 84.475) (end 101.7853 102.6353) (width 0.2) (layer "F.Cu") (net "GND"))
 (segment (start 101.7853 102.6353) (end 102.61 103.46) (width 0.2) (layer "F.Cu") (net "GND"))
 (segment (start 106.32 79.9403) (end 101.7853 84.475) (width 0.2) (layer "F.Cu") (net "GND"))
 (segment (start 115.6746 121.6472) (end 115.687 121.6472) (width 0.2) (layer "B.Cu") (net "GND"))
 (segment (start 133.25 79) (end 128.25 84) (width 0.2) (layer "B.Cu") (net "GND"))
 (segment (start 118.794 103.46) (end 118.61 103.46) (width 0.2) (layer "B.Cu") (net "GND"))
 (segment (start 115.6994 121.6472) (end 118.794 118.5526) (width 0.2) (layer "B.Cu") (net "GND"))
 (segment (start 135.1783 103.4483) (end 118.8057 103.4483) (width 0.2) (layer "B.Cu") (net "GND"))
 (segment (start 115.6498 121.6472) (end 115.6746 121.6472) (width 0.2) (layer "B.Cu") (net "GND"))
 (segment (start 115.6 121.6472) (end 115.6498 121.6472) (width 0.2) (layer "B.Cu") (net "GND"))
 (segment (start 118.5387 103.3887) (end 118.61 103.46) (width 0.2) (layer "B.Cu") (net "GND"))
 (segment (start 118.8057 103.4483) (end 118.794 103.46) (width 0.2) (layer "B.Cu") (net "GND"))
 (segment (start 115.687 121.6472) (end 115.6994 121.6472) (width 0.2) (layer "B.Cu") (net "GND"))
 (segment (start 142.75 79) (end 133.25 79) (width 0.2) (layer "B.Cu") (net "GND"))
 (segment (start 102.6813 103.3887) (end 118.5387 103.3887) (width 0.2) (layer "B.Cu") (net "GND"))
 (segment (start 135.19 103.46) (end 135.1783 103.4483) (width 0.2) (layer "B.Cu") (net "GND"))
 (segment (start 118.794 118.5526) (end 118.794 103.46) (width 0.2) (layer "B.Cu") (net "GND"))
 (segment (start 102.61 103.46) (end 102.6813 103.3887) (width 0.2) (layer "B.Cu") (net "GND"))
 (segment (start 106.6 120.1472) (end 106.99 120.1472) (width 0.2) (layer "B.Cu") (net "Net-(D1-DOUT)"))
 (segment (start 106.99 120.1472) (end 108.49 121.6472) (width 0.2) (layer "B.Cu") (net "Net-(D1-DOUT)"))
 (segment (start 108.49 121.6472) (end 110.4 121.6472) (width 0.2) (layer "B.Cu") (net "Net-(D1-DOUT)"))
 (segment (start 110.4 120.1472) (end 109.1681 118.9153) (width 0.2) (layer "B.Cu") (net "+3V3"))
 (segment (start 102.38 118.9153) (end 101.4 119.8953) (width 0.2) (layer "B.Cu") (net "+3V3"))
 (segment (start 101.4 119.8953) (end 101.4 120.1472) (width 0.2) (layer "B.Cu") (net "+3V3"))
 (segment (start 115.9356 103.5269) (end 115.9356 119.2066) (width 0.2) (layer "F.Cu") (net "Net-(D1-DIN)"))
 (segment (start 119.02 94.6) (end 119.02 100.4425) (width 0.2) (layer "F.Cu") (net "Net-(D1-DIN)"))
 (segment (start 119.02 100.4425) (end 115.9356 103.5269) (width 0.2) (layer "F.Cu") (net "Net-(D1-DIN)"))
 (via (at 115.9356 119.2066) (size 0.6) (drill 0.3) (layers "F.Cu" "B.Cu") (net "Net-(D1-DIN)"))
 (segment (start 115.6 120.1472) (end 115.9356 119.8116) (width 0.2) (layer "B.Cu") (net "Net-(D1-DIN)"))
 (segment (start 115.9356 119.8116) (end 115.9356 119.2066) (width 0.2) (layer "B.Cu") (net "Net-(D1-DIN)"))
 (segment (start 111.4 77.6) (end 111.4 79.3104) (width 0.2) (layer "F.Cu") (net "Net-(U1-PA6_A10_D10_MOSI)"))
 (segment (start 107.4411 100.92) (end 108.96 100.92) (width 0.2) (layer "F.Cu") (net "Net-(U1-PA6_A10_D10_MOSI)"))
 (segment (start 102.4539 95.9328) (end 107.4411 100.92) (width 0.2) (layer "F.Cu") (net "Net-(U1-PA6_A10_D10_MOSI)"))
 (segment (start 102.4539 93.2762) (end 102.4539 95.9328) (width 0.2) (layer "F.Cu") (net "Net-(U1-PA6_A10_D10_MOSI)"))
 (segment (start 111.4 79.3104) (end 106.6285 84.0819) (width 0.2) (layer "F.Cu") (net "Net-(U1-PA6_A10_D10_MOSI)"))
 (segment (start 106.6285 89.1016) (end 102.4539 93.2762) (width 0.2) (layer "F.Cu") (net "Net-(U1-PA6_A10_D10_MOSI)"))
 (segment (start 106.6285 84.0819) (end 106.6285 89.1016) (width 0.2) (layer "F.Cu") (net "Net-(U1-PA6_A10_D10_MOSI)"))
 (segment (start 124.96 100.92) (end 124.96 91.7309) (width 0.2) (layer "F.Cu") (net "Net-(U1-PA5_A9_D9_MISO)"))
 (segment (start 113.94 80.7109) (end 113.94 77.6) (width 0.2) (layer "F.Cu") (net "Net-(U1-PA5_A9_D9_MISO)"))
 (segment (start 124.96 91.7309) (end 113.94 80.7109) (width 0.2) (layer "F.Cu") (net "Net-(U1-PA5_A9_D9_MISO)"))
 (segment (start 125.3857 79.4376) (end 127.125 77.6983) (width 0.2) (layer "F.Cu") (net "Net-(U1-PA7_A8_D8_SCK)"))
 (segment (start 127.125 77.6983) (end 129.375 77.6983) (width 0.2) (layer "F.Cu") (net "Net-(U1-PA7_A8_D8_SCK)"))
 (segment (start 141.54 89.8633) (end 141.54 100.92) (width 0.2) (layer "F.Cu") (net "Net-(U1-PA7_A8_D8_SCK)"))
 (segment (start 116.48 77.6) (end 116.48 77.7126) (width 0.2) (layer "F.Cu") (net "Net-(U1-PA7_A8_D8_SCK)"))
 (segment (start 116.48 77.7126) (end 118.205 79.4376) (width 0.2) (layer "F.Cu") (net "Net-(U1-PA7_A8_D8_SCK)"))
 (segment (start 118.205 79.4376) (end 125.3857 79.4376) (width 0.2) (layer "F.Cu") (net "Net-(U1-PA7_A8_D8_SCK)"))
 (segment (start 129.375 77.6983) (end 141.54 89.8633) (width 0.2) (layer "F.Cu") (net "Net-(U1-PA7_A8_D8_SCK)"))
 (segment (start 108.86 94.6) (end 108.86 92.5895) (width 0.2) (layer "F.Cu") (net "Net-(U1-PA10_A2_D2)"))
 (via (at 108.86 92.5895) (size 0.6) (drill 0.3) (layers "F.Cu" "B.Cu") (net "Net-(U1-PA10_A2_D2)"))
 (segment (start 142.75 84) (end 134.1605 92.5895) (width 0.2) (layer "B.Cu") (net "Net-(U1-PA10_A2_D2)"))
 (segment (start 134.1605 92.5895) (end 108.86 92.5895) (width 0.2) (layer "B.Cu") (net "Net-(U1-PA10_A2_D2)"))
 (segment (start 104.978 92.8273) (end 103.78 94.0253) (width 0.2) (layer "F.Cu") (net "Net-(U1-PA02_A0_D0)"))
 (segment (start 103.78 94.0253) (end 103.78 94.6) (width 0.2) (layer "F.Cu") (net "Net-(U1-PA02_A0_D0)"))
 (via (at 104.978 92.8273) (size 0.6) (drill 0.3) (layers "F.Cu" "B.Cu") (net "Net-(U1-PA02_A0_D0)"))
 (segment (start 128.25 79) (end 118.8053 79) (width 0.2) (layer "B.Cu") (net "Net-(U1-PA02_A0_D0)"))
 (segment (start 118.8053 79) (end 104.978 92.8273) (width 0.2) (layer "B.Cu") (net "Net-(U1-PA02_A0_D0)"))
 (segment (start 106.32 94.1939) (end 106.32 94.6) (width 0.2) (layer "F.Cu") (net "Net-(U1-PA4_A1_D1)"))
 (segment (start 107.6105 92.9034) (end 106.32 94.1939) (width 0.2) (layer "F.Cu") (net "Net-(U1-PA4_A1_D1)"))
 (via (at 107.6105 92.9034) (size 0.6) (drill 0.3) (layers "F.Cu" "B.Cu") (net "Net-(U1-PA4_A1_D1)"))
 (segment (start 119.0139 81.5) (end 107.6105 92.9034) (width 0.2) (layer "B.Cu") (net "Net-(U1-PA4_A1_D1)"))
 (segment (start 128.25 81.5) (end 119.0139 81.5) (width 0.2) (layer "B.Cu") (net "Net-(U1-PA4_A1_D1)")))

